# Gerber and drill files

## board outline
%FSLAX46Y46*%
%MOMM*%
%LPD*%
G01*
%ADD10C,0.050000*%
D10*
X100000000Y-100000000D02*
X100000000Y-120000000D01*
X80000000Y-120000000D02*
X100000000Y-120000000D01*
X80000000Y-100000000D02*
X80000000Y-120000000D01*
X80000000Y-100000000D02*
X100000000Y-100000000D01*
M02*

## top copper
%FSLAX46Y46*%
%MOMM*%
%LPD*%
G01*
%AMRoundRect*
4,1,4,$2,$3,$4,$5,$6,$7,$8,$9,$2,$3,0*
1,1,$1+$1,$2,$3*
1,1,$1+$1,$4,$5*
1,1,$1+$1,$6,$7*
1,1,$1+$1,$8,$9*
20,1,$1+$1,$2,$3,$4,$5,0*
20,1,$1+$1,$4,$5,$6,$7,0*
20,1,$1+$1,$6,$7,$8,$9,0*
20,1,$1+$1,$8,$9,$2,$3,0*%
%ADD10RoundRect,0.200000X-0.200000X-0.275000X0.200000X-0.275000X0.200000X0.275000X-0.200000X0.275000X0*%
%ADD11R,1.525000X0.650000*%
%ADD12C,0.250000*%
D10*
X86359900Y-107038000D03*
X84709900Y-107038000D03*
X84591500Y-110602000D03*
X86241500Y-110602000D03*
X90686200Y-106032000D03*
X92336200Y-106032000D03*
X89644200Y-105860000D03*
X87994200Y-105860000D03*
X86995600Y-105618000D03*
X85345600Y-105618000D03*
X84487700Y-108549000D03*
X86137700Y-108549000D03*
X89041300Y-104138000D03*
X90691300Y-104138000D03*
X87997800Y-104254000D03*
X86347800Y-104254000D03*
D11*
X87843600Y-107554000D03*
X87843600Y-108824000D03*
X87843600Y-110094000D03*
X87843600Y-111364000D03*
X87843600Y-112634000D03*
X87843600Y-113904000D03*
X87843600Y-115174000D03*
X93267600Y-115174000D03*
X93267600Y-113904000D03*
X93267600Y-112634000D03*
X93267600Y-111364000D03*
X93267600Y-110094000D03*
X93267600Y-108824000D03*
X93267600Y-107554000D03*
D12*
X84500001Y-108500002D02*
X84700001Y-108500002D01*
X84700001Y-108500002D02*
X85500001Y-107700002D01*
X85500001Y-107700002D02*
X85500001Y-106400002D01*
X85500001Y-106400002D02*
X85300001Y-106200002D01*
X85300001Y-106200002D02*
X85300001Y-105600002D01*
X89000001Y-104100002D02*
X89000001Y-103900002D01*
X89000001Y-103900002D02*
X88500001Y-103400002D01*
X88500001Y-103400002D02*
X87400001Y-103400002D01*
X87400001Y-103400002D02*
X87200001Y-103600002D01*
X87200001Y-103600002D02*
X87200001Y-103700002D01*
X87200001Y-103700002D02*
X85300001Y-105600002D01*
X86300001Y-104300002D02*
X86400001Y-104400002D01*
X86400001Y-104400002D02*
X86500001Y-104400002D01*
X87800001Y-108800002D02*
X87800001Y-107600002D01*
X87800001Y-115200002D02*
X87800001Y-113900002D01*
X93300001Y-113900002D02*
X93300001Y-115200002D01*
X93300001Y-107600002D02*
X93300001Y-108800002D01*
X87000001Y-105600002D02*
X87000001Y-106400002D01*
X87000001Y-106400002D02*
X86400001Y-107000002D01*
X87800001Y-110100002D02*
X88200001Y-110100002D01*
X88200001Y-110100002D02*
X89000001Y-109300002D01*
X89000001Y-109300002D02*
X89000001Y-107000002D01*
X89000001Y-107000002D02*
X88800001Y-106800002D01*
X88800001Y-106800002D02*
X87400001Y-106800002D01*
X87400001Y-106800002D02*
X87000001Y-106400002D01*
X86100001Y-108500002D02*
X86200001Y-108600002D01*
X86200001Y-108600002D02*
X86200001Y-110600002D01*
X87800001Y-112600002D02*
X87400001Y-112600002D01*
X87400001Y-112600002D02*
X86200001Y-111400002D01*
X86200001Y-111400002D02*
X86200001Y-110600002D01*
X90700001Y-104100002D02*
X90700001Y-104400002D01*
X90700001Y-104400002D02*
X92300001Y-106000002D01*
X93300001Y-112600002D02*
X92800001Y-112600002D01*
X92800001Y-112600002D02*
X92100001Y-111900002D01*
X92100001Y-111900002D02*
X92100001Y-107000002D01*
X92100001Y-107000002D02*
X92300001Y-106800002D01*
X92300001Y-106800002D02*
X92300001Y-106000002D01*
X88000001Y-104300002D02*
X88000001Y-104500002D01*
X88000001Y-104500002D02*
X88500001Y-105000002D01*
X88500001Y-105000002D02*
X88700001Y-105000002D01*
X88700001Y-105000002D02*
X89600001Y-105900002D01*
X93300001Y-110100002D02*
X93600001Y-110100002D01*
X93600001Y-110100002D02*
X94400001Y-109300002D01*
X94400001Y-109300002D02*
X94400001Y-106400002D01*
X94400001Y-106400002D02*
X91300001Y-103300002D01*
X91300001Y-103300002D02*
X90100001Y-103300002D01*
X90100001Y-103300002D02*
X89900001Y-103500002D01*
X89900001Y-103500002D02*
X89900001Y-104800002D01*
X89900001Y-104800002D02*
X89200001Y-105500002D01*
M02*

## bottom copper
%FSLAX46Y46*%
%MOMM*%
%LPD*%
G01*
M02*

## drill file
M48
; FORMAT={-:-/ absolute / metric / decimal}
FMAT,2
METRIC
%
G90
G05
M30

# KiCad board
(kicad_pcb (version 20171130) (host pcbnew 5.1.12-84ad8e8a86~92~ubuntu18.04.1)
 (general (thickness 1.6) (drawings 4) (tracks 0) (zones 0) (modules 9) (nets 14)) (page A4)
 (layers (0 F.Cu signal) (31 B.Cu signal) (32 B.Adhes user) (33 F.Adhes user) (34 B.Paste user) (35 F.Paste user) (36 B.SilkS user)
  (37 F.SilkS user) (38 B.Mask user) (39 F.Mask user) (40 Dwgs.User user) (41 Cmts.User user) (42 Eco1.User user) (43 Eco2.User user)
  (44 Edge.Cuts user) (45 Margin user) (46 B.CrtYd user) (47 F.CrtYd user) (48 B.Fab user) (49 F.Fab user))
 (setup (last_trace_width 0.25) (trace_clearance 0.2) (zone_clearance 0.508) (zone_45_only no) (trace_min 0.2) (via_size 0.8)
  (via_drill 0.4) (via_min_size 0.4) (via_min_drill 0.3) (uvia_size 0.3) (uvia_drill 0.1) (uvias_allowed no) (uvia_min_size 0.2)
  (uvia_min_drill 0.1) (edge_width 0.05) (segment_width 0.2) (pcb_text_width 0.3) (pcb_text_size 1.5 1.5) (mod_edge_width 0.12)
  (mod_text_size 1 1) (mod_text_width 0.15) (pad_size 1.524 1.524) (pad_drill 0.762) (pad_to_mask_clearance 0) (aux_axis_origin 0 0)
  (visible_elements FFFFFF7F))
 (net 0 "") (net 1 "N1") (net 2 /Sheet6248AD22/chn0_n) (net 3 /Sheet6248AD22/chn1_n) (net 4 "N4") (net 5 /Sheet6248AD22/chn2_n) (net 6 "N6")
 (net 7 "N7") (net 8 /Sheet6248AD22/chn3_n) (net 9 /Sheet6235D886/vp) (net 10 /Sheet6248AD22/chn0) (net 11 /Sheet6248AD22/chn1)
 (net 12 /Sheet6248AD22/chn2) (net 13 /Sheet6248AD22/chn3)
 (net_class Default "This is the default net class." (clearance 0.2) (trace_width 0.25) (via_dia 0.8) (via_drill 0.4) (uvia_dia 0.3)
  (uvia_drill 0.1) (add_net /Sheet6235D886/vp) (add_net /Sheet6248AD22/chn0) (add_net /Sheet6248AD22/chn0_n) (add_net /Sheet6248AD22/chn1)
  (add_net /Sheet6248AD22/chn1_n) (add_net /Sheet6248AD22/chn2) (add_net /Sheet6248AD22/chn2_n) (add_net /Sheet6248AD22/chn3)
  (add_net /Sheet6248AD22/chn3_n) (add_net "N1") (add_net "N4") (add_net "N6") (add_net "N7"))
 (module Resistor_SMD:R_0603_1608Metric (layer F.Cu) (at 85.534900 107.038000)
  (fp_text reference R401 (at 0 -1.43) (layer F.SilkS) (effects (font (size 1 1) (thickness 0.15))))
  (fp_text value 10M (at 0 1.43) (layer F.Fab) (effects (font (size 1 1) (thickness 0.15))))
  (pad 2 smd roundrect (at 0.825 0) (size 0.8 0.95) (layers F.Cu F.Mask F.Paste) (roundrect_rratio 0.25) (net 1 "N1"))
  (pad 1 smd roundrect (at -0.825 0) (size 0.8 0.95) (layers F.Cu F.Mask F.Paste) (roundrect_rratio 0.25) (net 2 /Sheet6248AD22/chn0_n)))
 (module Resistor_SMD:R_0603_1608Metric (layer F.Cu) (at 85.416500 110.602000)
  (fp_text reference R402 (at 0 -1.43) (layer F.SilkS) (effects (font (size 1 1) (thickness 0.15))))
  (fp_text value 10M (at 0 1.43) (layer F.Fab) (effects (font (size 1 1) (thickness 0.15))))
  (pad 1 smd roundrect (at -0.825 0) (size 0.8 0.95) (layers F.Cu F.Mask F.Paste) (roundrect_rratio 0.25) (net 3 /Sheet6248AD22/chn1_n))
  (pad 2 smd roundrect (at 0.825 0) (size 0.8 0.95) (layers F.Cu F.Mask F.Paste) (roundrect_rratio 0.25) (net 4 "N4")))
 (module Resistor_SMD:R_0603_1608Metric (layer F.Cu) (at 91.511200 106.032000)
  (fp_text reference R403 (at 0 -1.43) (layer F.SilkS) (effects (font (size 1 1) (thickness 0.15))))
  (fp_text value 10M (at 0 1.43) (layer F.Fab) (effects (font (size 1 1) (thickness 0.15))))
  (pad 1 smd roundrect (at -0.825 0) (size 0.8 0.95) (layers F.Cu F.Mask F.Paste) (roundrect_rratio 0.25) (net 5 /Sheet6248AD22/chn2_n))
  (pad 2 smd roundrect (at 0.825 0) (size 0.8 0.95) (layers F.Cu F.Mask F.Paste) (roundrect_rratio 0.25) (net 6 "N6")))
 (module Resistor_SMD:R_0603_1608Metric (layer F.Cu) (at 88.819200 105.860000)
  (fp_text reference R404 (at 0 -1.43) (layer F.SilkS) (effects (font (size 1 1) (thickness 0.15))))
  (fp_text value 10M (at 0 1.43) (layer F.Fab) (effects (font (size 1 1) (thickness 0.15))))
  (pad 2 smd roundrect (at 0.825 0) (size 0.8 0.95) (layers F.Cu F.Mask F.Paste) (roundrect_rratio 0.25) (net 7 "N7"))
  (pad 1 smd roundrect (at -0.825 0) (size 0.8 0.95) (layers F.Cu F.Mask F.Paste) (roundrect_rratio 0.25) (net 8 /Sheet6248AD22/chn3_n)))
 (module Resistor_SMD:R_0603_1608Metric (layer F.Cu) (at 86.170600 105.618000)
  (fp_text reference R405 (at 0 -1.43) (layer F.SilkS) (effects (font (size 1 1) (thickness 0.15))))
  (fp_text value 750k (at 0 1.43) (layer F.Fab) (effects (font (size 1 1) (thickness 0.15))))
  (pad 2 smd roundrect (at 0.825 0) (size 0.8 0.95) (layers F.Cu F.Mask F.Paste) (roundrect_rratio 0.25) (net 1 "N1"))
  (pad 1 smd roundrect (at -0.825 0) (size 0.8 0.95) (layers F.Cu F.Mask F.Paste) (roundrect_rratio 0.25) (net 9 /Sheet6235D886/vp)))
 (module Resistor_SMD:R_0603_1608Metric (layer F.Cu) (at 85.312700 108.549000)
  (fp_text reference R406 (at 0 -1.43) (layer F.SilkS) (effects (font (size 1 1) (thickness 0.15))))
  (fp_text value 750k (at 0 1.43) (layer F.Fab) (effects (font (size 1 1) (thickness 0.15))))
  (pad 1 smd roundrect (at -0.825 0) (size 0.8 0.95) (layers F.Cu F.Mask F.Paste) (roundrect_rratio 0.25) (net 9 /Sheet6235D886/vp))
  (pad 2 smd roundrect (at 0.825 0) (size 0.8 0.95) (layers F.Cu F.Mask F.Paste) (roundrect_rratio 0.25) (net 4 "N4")))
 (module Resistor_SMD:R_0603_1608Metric (layer F.Cu) (at 89.866300 104.138000)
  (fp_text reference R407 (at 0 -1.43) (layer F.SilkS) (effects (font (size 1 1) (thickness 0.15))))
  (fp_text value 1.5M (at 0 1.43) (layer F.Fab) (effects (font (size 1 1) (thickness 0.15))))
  (pad 1 smd roundrect (at -0.825 0) (size 0.8 0.95) (layers F.Cu F.Mask F.Paste) (roundrect_rratio 0.25) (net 9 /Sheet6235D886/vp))
  (pad 2 smd roundrect (at 0.825 0) (size 0.8 0.95) (layers F.Cu F.Mask F.Paste) (roundrect_rratio 0.25) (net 6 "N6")))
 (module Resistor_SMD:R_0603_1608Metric (layer F.Cu) (at 87.172800 104.254000)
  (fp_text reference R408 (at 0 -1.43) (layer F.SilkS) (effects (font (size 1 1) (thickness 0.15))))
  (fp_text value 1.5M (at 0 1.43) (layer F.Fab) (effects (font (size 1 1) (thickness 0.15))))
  (pad 2 smd roundrect (at 0.825 0) (size 0.8 0.95) (layers F.Cu F.Mask F.Paste) (roundrect_rratio 0.25) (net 7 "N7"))
  (pad 1 smd roundrect (at -0.825 0) (size 0.8 0.95) (layers F.Cu F.Mask F.Paste) (roundrect_rratio 0.25) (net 9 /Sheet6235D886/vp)))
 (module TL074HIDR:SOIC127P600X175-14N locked (layer F.Cu) (at 90.555600 111.364000)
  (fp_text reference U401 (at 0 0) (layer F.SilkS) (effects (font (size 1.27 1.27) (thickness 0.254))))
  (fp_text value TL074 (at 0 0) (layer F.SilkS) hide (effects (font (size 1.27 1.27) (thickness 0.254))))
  (pad 1 smd rect (at -2.712 -3.81 90.000000) (size 0.65 1.525) (layers F.Cu F.Mask F.Paste) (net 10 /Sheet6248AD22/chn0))
  (pad 2 smd rect (at -2.712 -2.54 90.000000) (size 0.65 1.525) (layers F.Cu F.Mask F.Paste) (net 10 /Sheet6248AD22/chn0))
  (pad 3 smd rect (at -2.712 -1.27 90.000000) (size 0.65 1.525) (layers F.Cu F.Mask F.Paste) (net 1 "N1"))
  (pad 4 smd rect (at -2.712 0 90.000000) (size 0.65 1.525) (layers F.Cu F.Mask F.Paste))
  (pad 5 smd rect (at -2.712 1.27 90.000000) (size 0.65 1.525) (layers F.Cu F.Mask F.Paste) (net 4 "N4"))
  (pad 6 smd rect (at -2.712 2.54 90.000000) (size 0.65 1.525) (layers F.Cu F.Mask F.Paste) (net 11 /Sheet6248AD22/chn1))
  (pad 7 smd rect (at -2.712 3.81 90.000000) (size 0.65 1.525) (layers F.Cu F.Mask F.Paste) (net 11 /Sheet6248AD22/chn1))
  (pad 8 smd rect (at 2.712 3.81 90.000000) (size 0.65 1.525) (layers F.Cu F.Mask F.Paste) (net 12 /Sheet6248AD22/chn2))
  (pad 9 smd rect (at 2.712 2.54 90.000000) (size 0.65 1.525) (layers F.Cu F.Mask F.Paste) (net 12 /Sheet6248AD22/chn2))
  (pad 10 smd rect (at 2.712 1.27 90.000000) (size 0.65 1.525) (layers F.Cu F.Mask F.Paste) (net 6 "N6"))
  (pad 11 smd rect (at 2.712 0 90.000000) (size 0.65 1.525) (layers F.Cu F.Mask F.Paste))
  (pad 12 smd rect (at 2.712 -1.27 90.000000) (size 0.65 1.525) (layers F.Cu F.Mask F.Paste) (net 7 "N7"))
  (pad 13 smd rect (at 2.712 -2.54 90.000000) (size 0.65 1.525) (layers F.Cu F.Mask F.Paste) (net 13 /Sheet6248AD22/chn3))
  (pad 14 smd rect (at 2.712 -3.81 90.000000) (size 0.65 1.525) (layers F.Cu F.Mask F.Paste) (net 13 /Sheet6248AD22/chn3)))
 (gr_line (start 100 100) (end 100 120) (layer Edge.Cuts) (width 0.05))
 (gr_line (start 80 120) (end 100 120) (layer Edge.Cuts) (width 0.05))
 (gr_line (start 80 100) (end 80 120) (layer Edge.Cuts) (width 0.05))
 (gr_line (start 80 100) (end 100 100) (layer Edge.Cuts) (width 0.05))
 (segment (start 84.500001 108.500002) (end 84.700001 108.500002) (width 0.250000) (layer F.Cu) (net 9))
 (segment (start 84.700001 108.500002) (end 85.500001 107.700002) (width 0.250000) (layer F.Cu) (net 9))
 (segment (start 85.500001 107.700002) (end 85.500001 106.400002) (width 0.250000) (layer F.Cu) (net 9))
 (segment (start 85.500001 106.400002) (end 85.300001 106.200002) (width 0.250000) (layer F.Cu) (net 9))
 (segment (start 85.300001 106.200002) (end 85.300001 105.600002) (width 0.250000) (layer F.Cu) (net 9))
 (segment (start 89.000001 104.100002) (end 89.000001 103.900002) (width 0.250000) (layer F.Cu) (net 9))
 (segment (start 89.000001 103.900002) (end 88.500001 103.400002) (width 0.250000) (layer F.Cu) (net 9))
 (segment (start 88.500001 103.400002) (end 87.400001 103.400002) (width 0.250000) (layer F.Cu) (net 9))
 (segment (start 87.400001 103.400002) (end 87.200001 103.600002) (width 0.250000) (layer F.Cu) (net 9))
 (segment (start 87.200001 103.600002) (end 87.200001 103.700002) (width 0.250000) (layer F.Cu) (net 9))
 (segment (start 87.200001 103.700002) (end 85.300001 105.600002) (width 0.250000) (layer F.Cu) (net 9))
 (segment (start 86.300001 104.300002) (end 86.400001 104.400002) (width 0.250000) (layer F.Cu) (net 9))
 (segment (start 86.400001 104.400002) (end 86.500001 104.400002) (width 0.250000) (layer F.Cu) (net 9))
 (segment (start 87.800001 108.800002) (end 87.800001 107.600002) (width 0.250000) (layer F.Cu) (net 10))
 (segment (start 87.800001 115.200002) (end 87.800001 113.900002) (width 0.250000) (layer F.Cu) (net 11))
 (segment (start 93.300001 113.900002) (end 93.300001 115.200002) (width 0.250000) (layer F.Cu) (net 12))
 (segment (start 93.300001 107.600002) (end 93.300001 108.800002) (width 0.250000) (layer F.Cu) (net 13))
 (segment (start 87.000001 105.600002) (end 87.000001 106.400002) (width 0.250000) (layer F.Cu) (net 1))
 (segment (start 87.000001 106.400002) (end 86.400001 107.000002) (width 0.250000) (layer F.Cu) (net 1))
 (segment (start 87.800001 110.100002) (end 88.200001 110.100002) (width 0.250000) (layer F.Cu) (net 1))
 (segment (start 88.200001 110.100002) (end 89.000001 109.300002) (width 0.250000) (layer F.Cu) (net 1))
 (segment (start 89.000001 109.300002) (end 89.000001 107.000002) (width 0.250000) (layer F.Cu) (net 1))
 (segment (start 89.000001 107.000002) (end 88.800001 106.800002) (width 0.250000) (layer F.Cu) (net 1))
 (segment (start 88.800001 106.800002) (end 87.400001 106.800002) (width 0.250000) (layer F.Cu) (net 1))
 (segment (start 87.400001 106.800002) (end 87.000001 106.400002) (width 0.250000) (layer F.Cu) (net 1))
 (segment (start 86.100001 108.500002) (end 86.200001 108.600002) (width 0.250000) (layer F.Cu) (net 4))
 (segment (start 86.200001 108.600002) (end 86.200001 110.600002) (width 0.250000) (layer F.Cu) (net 4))
 (segment (start 87.800001 112.600002) (end 87.400001 112.600002) (width 0.250000) (layer F.Cu) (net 4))
 (segment (start 87.400001 112.600002) (end 86.200001 111.400002) (width 0.250000) (layer F.Cu) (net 4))
 (segment (start 86.200001 111.400002) (end 86.200001 110.600002) (width 0.250000) (layer F.Cu) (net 4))
 (segment (start 90.700001 104.100002) (end 90.700001 104.400002) (width 0.250000) (layer F.Cu) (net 6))
 (segment (start 90.700001 104.400002) (end 92.300001 106.000002) (width 0.250000) (layer F.Cu) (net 6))
 (segment (start 93.300001 112.600002) (end 92.800001 112.600002) (width 0.250000) (layer F.Cu) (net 6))
 (segment (start 92.800001 112.600002) (end 92.100001 111.900002) (width 0.250000) (layer F.Cu) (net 6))
 (segment (start 92.100001 111.900002) (end 92.100001 107.000002) (width 0.250000) (layer F.Cu) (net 6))
 (segment (start 92.100001 107.000002) (end 92.300001 106.800002) (width 0.250000) (layer F.Cu) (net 6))
 (segment (start 92.300001 106.800002) (end 92.300001 106.000002) (width 0.250000) (layer F.Cu) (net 6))
 (segment (start 88.000001 104.300002) (end 88.000001 104.500002) (width 0.250000) (layer F.Cu) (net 7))
 (segment (start 88.000001 104.500002) (end 88.500001 105.000002) (width 0.250000) (layer F.Cu) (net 7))
 (segment (start 88.500001 105.000002) (end 88.700001 105.000002) (width 0.250000) (layer F.Cu) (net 7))
 (segment (start 88.700001 105.000002) (end 89.600001 105.900002) (width 0.250000) (layer F.Cu) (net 7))
 (segment (start 93.300001 110.100002) (end 93.600001 110.100002) (width 0.250000) (layer F.Cu) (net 7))
 (segment (start 93.600001 110.100002) (end 94.400001 109.300002) (width 0.250000) (layer F.Cu) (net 7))
 (segment (start 94.400001 109.300002) (end 94.400001 106.400002) (width 0.250000) (layer F.Cu) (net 7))
 (segment (start 94.400001 106.400002) (end 91.300001 103.300002) (width 0.250000) (layer F.Cu) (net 7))
 (segment (start 91.300001 103.300002) (end 90.100001 103.300002) (width 0.250000) (layer F.Cu) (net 7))
 (segment (start 90.100001 103.300002) (end 89.900001 103.500002) (width 0.250000) (layer F.Cu) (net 7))
 (segment (start 89.900001 103.500002) (end 89.900001 104.800002) (width 0.250000) (layer F.Cu) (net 7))
 (segment (start 89.900001 104.800002) (end 89.200001 105.500002) (width 0.250000) (layer F.Cu) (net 7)))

